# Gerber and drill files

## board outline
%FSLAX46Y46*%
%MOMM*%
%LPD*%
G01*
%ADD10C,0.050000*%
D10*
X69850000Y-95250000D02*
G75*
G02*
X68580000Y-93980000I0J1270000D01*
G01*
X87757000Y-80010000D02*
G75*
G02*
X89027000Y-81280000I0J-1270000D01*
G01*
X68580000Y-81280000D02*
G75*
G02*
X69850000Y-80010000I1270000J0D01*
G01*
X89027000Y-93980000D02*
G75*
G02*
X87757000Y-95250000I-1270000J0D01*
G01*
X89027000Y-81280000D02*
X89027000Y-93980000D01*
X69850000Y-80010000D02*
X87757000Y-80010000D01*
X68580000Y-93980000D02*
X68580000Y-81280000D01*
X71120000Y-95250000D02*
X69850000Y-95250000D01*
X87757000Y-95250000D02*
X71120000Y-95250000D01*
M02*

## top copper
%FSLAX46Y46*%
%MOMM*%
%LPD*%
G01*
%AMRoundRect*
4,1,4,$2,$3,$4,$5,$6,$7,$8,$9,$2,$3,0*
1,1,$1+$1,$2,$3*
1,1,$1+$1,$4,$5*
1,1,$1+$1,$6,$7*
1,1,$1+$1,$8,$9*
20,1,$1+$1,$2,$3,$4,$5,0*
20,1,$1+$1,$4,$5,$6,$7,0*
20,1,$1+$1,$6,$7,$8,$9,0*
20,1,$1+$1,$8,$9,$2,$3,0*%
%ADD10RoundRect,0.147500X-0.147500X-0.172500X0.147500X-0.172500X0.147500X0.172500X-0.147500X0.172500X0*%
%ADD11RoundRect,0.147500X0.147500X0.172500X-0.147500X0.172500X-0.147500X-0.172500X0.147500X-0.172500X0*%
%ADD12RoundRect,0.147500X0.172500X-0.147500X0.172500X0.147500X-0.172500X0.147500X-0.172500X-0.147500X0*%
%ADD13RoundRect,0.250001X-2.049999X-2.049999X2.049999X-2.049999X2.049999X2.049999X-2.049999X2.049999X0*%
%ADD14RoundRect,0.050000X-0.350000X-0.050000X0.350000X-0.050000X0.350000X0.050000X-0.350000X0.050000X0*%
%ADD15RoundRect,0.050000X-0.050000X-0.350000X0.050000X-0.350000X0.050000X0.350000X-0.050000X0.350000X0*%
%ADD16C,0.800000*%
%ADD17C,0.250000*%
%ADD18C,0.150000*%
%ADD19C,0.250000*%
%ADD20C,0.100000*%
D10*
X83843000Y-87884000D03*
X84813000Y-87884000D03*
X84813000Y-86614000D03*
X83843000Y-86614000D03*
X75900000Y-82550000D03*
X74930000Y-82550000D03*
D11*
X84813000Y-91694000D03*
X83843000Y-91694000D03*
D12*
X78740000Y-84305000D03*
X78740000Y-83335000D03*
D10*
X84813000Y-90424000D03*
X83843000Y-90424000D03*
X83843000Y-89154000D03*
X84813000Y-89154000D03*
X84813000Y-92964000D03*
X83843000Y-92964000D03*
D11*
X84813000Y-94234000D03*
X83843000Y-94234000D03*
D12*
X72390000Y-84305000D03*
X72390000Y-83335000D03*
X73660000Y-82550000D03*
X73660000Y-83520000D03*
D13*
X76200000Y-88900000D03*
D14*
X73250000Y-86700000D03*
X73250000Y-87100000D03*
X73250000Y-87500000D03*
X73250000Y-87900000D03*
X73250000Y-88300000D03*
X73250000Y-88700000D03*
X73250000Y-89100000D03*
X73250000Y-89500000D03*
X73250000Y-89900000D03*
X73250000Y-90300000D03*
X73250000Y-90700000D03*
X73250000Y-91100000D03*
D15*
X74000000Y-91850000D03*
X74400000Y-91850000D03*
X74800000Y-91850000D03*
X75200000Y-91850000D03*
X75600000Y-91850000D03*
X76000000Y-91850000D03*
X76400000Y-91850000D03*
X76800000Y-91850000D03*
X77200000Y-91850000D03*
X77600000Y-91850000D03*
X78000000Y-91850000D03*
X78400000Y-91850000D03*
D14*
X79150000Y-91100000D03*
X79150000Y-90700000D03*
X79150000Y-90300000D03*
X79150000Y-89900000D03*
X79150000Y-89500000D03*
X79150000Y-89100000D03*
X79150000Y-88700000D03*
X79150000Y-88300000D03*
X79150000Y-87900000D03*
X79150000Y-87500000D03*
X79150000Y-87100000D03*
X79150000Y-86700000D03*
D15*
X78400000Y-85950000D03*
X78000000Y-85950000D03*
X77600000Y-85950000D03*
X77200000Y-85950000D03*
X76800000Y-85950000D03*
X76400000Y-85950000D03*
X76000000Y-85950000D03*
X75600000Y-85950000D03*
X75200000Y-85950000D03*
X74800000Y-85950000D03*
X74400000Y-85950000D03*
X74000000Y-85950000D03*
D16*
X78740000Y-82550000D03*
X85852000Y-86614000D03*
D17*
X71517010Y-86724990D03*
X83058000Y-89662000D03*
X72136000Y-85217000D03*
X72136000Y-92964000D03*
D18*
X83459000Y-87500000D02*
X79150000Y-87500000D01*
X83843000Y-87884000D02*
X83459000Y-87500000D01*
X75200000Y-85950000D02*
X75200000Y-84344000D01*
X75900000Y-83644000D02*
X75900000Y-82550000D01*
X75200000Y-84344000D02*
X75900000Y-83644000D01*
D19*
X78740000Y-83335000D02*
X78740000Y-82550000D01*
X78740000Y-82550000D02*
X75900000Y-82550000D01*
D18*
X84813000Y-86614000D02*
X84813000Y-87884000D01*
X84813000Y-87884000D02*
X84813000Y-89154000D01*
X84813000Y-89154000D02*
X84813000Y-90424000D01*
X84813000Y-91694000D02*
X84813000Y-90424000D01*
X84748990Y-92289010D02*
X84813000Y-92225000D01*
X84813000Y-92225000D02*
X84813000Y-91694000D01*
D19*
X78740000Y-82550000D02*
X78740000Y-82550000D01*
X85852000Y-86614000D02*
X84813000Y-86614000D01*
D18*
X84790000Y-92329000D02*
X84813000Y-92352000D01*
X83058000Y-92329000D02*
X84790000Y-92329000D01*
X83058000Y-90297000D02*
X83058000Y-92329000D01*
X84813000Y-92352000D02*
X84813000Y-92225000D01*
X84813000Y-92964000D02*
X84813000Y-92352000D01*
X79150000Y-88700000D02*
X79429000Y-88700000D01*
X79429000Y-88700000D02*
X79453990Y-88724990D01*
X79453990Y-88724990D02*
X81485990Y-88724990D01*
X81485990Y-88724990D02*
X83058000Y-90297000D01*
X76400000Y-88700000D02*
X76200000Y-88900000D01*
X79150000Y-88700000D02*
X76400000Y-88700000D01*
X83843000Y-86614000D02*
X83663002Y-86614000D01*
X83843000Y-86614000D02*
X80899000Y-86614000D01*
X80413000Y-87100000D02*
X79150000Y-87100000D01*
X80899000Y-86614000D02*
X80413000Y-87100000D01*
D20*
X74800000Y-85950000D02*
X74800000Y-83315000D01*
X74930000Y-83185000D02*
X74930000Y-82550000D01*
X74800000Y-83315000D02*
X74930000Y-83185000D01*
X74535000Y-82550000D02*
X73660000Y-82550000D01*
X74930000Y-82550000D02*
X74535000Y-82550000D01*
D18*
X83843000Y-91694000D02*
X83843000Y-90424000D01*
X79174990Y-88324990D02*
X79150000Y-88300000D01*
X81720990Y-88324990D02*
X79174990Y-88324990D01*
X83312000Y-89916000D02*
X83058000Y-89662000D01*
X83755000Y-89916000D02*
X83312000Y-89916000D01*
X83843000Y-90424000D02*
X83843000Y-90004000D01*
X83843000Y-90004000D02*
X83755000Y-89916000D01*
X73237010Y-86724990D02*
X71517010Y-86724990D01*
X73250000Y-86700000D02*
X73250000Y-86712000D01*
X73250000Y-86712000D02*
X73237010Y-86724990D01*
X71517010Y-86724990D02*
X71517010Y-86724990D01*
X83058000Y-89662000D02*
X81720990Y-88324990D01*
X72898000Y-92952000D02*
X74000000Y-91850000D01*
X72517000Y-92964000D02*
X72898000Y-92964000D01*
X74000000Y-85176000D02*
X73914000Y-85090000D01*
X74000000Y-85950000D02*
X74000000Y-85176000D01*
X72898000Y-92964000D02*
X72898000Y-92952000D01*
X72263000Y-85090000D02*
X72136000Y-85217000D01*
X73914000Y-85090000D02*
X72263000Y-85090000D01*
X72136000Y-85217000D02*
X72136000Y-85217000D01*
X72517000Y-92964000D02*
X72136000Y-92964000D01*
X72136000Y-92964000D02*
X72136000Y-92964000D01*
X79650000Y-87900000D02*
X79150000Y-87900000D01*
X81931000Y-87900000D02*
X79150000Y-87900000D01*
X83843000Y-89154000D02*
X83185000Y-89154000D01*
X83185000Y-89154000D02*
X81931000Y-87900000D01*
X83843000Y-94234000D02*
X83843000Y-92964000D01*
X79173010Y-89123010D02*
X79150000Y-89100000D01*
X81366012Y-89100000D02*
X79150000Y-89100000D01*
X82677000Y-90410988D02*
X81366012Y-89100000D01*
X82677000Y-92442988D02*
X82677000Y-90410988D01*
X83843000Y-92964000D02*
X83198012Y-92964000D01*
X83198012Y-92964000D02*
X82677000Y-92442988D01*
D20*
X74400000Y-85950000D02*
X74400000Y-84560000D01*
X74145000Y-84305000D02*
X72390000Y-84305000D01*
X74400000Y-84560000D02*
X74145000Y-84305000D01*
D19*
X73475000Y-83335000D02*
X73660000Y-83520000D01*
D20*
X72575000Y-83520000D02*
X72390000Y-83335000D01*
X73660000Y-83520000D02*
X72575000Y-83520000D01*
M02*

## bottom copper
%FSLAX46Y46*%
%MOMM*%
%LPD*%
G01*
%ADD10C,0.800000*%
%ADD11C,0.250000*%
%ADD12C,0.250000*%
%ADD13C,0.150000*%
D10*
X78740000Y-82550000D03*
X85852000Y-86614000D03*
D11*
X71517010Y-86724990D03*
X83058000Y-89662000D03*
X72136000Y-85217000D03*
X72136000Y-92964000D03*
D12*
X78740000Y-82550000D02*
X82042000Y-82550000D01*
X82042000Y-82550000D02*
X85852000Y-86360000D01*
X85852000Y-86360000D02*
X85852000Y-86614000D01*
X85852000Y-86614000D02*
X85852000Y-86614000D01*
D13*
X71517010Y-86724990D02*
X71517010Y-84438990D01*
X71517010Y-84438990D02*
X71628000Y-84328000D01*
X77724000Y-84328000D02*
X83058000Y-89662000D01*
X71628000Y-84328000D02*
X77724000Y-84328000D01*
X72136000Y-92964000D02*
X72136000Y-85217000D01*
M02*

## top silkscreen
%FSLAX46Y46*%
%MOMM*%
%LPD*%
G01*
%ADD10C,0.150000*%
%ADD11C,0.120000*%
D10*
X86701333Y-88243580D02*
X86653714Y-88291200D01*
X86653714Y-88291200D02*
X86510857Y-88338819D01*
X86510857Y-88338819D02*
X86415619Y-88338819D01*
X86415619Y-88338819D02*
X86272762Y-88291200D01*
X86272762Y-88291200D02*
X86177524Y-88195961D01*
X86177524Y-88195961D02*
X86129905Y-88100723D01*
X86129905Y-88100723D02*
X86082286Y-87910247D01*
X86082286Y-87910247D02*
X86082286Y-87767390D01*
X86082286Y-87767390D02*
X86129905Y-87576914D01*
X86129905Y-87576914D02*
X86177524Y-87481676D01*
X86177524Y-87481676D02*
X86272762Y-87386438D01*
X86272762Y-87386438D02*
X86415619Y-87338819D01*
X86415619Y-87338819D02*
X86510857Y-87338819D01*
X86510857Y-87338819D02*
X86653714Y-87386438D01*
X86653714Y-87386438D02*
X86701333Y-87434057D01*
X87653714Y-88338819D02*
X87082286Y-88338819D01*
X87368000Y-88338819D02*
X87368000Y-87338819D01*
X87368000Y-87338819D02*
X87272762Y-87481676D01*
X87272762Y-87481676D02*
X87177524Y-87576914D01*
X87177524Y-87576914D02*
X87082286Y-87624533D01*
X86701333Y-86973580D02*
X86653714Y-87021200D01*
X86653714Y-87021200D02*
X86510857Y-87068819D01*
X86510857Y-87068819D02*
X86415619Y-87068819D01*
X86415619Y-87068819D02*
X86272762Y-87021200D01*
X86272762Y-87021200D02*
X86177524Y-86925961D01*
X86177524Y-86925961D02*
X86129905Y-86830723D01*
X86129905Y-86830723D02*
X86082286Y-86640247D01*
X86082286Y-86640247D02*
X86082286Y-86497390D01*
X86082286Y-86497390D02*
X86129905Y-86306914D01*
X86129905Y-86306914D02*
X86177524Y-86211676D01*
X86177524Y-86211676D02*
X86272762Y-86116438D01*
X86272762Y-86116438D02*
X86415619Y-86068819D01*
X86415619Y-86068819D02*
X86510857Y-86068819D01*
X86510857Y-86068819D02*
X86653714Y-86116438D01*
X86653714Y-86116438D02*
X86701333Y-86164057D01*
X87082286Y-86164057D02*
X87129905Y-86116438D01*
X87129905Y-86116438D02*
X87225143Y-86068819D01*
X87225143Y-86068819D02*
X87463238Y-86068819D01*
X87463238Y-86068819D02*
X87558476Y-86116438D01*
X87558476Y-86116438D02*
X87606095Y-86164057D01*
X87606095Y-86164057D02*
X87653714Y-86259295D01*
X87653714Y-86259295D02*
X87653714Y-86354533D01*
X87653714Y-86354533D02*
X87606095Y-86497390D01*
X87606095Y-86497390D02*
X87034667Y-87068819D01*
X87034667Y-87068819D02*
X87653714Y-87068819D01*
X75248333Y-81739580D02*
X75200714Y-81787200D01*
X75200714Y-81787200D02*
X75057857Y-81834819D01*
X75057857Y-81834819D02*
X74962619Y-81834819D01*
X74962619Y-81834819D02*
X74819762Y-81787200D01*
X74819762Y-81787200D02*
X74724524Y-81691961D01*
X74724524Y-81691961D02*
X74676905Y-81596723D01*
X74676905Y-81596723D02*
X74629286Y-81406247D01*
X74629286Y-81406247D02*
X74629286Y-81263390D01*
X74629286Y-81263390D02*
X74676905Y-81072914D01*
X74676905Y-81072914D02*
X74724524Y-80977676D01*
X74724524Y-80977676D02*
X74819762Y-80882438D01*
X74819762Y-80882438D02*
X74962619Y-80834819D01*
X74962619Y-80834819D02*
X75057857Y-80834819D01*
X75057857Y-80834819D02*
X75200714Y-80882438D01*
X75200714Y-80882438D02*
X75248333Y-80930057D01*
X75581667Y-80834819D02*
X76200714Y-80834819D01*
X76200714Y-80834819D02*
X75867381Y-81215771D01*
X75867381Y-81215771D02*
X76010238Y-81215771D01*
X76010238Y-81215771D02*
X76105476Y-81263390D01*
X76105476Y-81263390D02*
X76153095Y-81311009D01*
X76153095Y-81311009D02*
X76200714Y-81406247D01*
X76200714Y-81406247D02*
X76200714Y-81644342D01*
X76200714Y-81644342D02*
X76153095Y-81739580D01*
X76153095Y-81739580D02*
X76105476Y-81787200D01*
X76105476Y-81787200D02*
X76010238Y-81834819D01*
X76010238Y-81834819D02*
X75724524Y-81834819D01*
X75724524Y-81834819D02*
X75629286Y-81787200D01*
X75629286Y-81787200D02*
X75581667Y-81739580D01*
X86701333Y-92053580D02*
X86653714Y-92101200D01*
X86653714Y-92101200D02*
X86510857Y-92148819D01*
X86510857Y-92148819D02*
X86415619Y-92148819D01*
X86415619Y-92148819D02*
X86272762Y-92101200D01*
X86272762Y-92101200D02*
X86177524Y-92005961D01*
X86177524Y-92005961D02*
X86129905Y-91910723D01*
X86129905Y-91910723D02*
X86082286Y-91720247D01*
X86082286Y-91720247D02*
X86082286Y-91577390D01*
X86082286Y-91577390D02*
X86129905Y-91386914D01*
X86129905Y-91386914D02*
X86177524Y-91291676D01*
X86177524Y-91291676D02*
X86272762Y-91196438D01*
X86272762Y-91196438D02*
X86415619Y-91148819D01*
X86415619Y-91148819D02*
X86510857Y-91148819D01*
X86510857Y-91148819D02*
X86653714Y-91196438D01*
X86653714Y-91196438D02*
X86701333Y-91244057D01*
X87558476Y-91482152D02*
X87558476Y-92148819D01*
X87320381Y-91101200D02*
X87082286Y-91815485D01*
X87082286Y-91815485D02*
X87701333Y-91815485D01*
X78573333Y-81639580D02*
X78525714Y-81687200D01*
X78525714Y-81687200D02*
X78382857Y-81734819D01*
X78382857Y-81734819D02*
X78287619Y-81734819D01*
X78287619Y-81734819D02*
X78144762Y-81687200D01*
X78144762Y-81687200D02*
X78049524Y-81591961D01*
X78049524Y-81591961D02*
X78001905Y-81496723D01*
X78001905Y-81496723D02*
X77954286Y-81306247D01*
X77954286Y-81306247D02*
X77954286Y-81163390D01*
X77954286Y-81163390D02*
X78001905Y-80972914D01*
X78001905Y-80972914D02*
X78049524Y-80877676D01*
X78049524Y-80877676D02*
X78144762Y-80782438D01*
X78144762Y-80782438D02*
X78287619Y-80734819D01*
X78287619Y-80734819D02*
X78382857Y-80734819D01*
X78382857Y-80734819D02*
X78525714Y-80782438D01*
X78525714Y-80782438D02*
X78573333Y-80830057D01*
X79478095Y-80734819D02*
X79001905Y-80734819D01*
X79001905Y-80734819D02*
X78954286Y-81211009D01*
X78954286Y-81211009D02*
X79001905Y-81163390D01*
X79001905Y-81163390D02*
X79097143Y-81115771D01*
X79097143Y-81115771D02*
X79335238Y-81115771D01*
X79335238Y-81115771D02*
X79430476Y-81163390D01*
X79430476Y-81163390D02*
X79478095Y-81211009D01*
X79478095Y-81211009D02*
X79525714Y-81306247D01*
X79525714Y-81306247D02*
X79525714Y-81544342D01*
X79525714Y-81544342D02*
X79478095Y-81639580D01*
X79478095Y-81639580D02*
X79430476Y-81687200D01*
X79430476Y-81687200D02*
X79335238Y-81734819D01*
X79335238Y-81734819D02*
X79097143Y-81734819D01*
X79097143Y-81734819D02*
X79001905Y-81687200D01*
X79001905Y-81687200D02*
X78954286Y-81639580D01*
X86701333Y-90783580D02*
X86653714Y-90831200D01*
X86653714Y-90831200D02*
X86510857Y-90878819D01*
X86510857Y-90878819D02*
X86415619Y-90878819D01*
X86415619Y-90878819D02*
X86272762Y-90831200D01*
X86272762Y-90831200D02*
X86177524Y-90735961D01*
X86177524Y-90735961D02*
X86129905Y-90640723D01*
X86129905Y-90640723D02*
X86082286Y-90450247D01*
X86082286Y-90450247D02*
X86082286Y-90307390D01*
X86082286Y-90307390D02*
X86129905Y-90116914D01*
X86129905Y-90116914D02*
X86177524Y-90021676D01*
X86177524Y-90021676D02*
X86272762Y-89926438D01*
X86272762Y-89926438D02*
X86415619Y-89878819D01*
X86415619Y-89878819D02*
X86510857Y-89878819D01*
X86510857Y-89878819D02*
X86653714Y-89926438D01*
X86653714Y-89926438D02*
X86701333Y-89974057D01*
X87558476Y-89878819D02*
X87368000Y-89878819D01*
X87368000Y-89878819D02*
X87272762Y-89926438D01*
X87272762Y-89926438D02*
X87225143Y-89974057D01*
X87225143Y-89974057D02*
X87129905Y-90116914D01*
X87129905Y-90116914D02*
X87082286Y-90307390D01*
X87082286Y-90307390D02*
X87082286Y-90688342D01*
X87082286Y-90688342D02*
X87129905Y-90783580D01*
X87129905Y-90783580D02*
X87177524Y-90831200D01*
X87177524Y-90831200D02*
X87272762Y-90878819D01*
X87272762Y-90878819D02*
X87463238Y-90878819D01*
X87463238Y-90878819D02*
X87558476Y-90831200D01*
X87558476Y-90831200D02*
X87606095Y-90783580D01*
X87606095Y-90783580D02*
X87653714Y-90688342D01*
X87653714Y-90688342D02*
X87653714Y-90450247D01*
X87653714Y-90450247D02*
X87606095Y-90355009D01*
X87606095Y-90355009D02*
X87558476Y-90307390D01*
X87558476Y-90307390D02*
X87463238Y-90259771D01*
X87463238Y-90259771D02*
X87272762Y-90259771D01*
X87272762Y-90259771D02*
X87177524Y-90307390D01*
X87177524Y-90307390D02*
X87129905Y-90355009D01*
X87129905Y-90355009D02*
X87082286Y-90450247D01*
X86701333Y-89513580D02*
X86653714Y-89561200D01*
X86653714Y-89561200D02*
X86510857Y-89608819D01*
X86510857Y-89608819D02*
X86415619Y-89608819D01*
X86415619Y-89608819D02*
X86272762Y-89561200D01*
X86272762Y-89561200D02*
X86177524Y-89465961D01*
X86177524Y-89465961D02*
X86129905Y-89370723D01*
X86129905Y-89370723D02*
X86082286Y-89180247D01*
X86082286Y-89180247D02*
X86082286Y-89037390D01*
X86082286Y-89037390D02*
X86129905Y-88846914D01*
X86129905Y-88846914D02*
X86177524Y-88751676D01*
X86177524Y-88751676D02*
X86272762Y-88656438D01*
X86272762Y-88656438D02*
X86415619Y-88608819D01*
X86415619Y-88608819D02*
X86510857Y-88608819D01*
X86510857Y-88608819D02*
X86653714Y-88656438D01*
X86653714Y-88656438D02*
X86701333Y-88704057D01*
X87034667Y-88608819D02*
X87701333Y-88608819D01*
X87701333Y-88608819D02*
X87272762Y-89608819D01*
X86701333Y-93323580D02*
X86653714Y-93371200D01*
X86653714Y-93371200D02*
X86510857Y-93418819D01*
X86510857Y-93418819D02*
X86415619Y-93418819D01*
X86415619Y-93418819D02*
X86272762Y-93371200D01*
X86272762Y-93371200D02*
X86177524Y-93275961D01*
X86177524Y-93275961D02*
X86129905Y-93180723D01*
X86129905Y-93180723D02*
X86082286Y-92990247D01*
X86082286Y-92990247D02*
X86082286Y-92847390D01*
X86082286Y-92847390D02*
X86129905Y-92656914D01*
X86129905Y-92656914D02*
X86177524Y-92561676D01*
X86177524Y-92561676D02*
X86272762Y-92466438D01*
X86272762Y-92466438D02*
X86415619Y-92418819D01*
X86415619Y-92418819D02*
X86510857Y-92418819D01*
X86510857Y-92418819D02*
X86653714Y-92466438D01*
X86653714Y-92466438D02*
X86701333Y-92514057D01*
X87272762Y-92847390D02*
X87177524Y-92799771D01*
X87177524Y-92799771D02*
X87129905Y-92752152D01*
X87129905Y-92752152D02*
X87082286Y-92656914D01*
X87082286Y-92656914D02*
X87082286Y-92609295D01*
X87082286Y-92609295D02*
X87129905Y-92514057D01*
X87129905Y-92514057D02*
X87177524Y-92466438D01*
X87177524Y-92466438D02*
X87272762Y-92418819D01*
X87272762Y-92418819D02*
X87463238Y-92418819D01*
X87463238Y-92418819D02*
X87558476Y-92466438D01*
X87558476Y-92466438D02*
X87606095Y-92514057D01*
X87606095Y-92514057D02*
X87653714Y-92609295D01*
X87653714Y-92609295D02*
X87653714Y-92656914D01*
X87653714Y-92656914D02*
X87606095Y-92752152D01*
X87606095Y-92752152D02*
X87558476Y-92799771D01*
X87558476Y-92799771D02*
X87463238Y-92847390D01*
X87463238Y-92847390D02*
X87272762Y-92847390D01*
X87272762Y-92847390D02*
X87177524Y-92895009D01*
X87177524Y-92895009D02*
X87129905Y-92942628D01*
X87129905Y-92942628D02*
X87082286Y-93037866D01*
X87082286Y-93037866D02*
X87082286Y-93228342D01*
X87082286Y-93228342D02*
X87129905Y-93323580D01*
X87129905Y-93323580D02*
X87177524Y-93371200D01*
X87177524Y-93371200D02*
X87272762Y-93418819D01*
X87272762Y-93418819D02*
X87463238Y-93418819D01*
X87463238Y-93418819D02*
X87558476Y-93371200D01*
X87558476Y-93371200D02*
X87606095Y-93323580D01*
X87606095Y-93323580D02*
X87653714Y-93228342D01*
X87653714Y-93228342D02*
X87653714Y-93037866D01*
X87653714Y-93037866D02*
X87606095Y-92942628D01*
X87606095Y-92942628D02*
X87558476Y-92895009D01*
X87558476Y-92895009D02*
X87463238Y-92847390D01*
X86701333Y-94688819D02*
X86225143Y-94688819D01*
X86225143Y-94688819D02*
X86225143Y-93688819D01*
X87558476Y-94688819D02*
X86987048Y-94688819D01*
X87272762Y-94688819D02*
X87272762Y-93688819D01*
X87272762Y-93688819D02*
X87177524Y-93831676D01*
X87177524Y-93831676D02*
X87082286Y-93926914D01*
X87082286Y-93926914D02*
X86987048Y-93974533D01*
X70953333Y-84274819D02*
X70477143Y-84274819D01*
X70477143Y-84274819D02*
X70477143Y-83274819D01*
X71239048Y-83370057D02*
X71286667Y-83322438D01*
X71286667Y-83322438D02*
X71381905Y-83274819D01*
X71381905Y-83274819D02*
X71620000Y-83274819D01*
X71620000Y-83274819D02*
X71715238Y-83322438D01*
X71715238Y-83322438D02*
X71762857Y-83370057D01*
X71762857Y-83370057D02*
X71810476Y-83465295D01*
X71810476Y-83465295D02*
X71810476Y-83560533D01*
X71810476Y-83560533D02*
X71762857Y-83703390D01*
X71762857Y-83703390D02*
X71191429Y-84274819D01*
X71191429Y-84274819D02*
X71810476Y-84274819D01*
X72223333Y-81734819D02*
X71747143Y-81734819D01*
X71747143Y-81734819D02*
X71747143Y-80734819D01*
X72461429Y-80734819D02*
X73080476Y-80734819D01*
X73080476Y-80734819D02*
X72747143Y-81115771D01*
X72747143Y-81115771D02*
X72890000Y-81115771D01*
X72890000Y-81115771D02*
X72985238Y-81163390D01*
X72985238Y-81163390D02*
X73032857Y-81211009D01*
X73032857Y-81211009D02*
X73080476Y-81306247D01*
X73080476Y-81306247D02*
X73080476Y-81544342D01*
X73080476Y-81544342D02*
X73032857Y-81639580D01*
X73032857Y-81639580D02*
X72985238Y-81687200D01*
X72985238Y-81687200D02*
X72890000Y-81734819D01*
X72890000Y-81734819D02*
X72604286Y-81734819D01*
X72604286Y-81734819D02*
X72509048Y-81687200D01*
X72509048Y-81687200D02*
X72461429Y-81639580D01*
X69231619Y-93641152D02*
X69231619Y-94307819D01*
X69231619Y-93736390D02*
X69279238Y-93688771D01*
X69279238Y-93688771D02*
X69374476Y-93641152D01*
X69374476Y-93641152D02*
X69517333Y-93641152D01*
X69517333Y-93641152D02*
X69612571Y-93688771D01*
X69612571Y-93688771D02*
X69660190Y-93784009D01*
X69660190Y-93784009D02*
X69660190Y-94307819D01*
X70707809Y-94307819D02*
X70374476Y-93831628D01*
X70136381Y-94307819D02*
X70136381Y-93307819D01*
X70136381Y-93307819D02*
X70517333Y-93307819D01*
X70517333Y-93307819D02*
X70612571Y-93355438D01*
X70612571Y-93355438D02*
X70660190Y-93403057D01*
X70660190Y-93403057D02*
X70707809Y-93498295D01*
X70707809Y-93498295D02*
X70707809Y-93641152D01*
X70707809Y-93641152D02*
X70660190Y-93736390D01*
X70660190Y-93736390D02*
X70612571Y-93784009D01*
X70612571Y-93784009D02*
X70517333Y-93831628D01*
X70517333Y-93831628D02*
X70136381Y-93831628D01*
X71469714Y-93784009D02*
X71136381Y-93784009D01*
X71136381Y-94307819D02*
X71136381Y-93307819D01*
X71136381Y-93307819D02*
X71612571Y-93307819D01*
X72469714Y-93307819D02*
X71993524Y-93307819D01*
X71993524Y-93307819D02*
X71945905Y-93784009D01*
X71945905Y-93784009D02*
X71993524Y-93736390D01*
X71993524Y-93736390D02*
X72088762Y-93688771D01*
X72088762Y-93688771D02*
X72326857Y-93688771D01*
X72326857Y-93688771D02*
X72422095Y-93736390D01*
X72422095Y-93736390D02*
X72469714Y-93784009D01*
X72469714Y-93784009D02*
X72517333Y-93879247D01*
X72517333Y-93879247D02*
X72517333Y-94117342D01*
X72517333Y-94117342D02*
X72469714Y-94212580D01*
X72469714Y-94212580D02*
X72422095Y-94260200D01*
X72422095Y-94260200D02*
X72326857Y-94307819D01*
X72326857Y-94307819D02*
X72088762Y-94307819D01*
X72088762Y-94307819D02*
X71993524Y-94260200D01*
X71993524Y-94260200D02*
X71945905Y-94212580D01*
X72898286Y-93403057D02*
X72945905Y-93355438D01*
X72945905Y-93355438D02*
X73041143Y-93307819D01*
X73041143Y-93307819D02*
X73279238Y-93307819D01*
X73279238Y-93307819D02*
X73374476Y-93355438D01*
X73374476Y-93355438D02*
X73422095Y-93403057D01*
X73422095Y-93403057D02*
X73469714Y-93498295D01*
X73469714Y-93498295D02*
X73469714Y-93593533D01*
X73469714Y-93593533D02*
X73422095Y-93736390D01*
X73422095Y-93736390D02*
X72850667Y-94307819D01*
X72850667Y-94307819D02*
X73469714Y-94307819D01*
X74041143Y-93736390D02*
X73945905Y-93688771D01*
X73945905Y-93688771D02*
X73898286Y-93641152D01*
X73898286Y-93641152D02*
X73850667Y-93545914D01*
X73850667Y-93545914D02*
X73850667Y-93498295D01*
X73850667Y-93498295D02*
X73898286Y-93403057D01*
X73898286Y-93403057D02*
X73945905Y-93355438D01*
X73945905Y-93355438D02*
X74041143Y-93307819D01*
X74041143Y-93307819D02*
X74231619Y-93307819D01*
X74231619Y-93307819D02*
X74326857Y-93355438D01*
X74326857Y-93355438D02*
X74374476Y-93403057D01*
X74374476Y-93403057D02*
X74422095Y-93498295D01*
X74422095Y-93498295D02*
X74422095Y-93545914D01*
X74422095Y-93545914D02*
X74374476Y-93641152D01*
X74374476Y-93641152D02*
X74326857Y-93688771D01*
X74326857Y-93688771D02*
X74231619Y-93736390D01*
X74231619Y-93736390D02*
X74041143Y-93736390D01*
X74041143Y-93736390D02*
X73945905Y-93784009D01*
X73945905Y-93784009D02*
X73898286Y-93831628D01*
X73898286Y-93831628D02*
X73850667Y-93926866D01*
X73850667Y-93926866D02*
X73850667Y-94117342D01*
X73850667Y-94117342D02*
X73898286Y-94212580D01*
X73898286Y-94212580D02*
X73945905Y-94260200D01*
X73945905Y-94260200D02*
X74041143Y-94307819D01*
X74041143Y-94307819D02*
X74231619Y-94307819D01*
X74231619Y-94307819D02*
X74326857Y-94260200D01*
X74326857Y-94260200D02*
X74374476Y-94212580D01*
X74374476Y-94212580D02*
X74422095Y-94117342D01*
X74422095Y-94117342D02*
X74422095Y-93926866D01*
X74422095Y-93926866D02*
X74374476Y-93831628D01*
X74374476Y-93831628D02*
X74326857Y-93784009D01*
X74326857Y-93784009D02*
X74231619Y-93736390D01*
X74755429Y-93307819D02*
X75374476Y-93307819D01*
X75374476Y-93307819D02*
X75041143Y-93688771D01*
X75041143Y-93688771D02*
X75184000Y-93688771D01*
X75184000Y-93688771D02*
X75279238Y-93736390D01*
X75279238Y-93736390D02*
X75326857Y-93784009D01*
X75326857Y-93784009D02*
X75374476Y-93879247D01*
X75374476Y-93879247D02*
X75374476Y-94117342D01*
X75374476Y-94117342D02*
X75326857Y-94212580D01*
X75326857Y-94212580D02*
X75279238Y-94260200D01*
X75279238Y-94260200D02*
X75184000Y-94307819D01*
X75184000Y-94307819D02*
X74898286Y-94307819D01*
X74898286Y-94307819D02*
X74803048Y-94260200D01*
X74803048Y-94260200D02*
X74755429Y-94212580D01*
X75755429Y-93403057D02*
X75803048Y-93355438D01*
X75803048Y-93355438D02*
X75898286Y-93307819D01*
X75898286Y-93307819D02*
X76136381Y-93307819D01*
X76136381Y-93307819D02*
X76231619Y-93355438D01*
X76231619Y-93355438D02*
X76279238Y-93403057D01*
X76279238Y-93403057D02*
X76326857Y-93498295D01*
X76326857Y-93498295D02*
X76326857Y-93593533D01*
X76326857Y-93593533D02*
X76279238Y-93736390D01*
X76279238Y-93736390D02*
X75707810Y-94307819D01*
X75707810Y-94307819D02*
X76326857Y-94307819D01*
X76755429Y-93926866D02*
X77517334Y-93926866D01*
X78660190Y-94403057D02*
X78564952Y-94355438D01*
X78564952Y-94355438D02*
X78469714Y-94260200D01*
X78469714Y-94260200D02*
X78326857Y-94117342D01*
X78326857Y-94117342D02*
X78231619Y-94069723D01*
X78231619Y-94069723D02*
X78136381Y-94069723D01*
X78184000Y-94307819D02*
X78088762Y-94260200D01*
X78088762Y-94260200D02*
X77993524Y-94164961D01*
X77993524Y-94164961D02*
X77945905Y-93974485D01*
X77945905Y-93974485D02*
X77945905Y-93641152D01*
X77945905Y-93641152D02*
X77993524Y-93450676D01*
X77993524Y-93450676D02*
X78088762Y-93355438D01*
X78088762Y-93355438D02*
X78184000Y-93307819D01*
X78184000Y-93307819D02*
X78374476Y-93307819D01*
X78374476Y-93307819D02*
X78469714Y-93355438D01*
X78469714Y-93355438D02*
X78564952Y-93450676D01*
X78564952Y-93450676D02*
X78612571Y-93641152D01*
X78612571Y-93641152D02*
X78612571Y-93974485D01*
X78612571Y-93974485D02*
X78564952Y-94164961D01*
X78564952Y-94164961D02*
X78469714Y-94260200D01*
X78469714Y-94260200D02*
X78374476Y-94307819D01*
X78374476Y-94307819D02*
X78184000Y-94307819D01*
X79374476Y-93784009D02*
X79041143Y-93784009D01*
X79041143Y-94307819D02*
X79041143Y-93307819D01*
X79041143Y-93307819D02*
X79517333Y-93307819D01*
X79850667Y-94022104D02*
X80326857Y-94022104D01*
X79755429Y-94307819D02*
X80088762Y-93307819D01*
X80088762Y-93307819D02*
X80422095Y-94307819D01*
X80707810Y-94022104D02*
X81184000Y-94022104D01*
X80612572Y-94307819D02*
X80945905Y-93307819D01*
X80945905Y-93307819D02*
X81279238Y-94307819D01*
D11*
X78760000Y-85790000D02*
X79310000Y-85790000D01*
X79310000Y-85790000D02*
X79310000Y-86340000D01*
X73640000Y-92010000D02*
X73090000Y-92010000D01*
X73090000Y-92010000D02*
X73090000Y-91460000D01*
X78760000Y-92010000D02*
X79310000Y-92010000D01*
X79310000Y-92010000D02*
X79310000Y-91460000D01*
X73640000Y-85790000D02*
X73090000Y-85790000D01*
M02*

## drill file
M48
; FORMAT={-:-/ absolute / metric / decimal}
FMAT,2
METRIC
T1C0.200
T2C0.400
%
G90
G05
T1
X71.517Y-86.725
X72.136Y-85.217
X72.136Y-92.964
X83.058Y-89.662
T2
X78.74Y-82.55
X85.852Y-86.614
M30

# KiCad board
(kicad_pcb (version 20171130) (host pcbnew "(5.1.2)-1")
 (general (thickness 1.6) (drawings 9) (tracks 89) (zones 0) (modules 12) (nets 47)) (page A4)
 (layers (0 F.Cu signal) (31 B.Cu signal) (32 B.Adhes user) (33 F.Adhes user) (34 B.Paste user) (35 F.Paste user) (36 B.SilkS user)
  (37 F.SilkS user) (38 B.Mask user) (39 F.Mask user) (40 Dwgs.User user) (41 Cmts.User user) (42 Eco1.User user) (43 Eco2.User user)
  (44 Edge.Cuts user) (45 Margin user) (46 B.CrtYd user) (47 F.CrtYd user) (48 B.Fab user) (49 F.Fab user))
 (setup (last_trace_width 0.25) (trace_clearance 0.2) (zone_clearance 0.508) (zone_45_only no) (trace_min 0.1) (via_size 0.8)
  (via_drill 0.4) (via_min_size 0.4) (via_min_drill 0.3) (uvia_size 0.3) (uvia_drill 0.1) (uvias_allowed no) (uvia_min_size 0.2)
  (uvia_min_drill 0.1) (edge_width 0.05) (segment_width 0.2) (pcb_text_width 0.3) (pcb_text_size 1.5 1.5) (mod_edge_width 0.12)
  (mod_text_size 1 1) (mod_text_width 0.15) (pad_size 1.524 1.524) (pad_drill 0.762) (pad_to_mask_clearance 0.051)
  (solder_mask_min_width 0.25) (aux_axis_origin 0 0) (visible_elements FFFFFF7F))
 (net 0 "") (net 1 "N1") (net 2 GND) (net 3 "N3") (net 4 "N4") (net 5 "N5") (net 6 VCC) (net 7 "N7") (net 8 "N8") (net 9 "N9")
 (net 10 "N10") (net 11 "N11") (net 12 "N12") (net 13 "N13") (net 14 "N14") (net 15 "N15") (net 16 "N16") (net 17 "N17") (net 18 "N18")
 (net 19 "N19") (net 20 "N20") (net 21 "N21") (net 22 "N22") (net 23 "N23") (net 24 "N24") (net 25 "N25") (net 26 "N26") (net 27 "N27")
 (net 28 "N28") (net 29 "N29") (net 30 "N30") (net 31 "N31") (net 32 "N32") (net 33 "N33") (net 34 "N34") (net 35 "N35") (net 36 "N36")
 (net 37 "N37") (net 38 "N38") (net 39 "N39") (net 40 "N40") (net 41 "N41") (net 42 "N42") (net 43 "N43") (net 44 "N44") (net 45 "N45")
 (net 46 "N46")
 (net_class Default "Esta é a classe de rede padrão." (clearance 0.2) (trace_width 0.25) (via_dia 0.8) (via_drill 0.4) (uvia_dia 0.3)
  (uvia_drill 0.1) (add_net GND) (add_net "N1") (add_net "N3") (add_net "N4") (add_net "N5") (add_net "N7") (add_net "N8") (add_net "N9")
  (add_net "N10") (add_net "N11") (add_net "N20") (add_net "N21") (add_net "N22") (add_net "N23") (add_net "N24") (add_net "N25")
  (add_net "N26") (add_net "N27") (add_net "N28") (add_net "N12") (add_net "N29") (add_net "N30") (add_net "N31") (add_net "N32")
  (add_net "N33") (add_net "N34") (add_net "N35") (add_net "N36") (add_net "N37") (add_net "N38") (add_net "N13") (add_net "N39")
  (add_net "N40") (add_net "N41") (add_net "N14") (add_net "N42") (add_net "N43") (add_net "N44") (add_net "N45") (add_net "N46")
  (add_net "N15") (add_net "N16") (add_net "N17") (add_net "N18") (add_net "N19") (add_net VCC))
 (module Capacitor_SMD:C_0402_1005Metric (layer F.Cu) (at 84.328 87.884)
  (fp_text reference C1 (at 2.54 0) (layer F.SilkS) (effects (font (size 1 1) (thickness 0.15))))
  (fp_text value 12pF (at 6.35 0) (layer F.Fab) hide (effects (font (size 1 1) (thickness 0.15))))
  (pad 1 smd roundrect (at -0.485 0) (size 0.59 0.64) (layers F.Cu F.Paste F.Mask) (roundrect_rratio 0.25) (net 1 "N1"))
  (pad 2 smd roundrect (at 0.485 0) (size 0.59 0.64) (layers F.Cu F.Paste F.Mask) (roundrect_rratio 0.25) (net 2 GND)))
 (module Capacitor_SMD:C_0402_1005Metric (layer F.Cu) (at 84.328 86.614)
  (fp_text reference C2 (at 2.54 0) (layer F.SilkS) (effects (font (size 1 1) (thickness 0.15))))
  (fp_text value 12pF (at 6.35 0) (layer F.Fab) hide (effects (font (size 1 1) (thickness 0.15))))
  (pad 2 smd roundrect (at 0.485 0) (size 0.59 0.64) (layers F.Cu F.Paste F.Mask) (roundrect_rratio 0.25) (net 2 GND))
  (pad 1 smd roundrect (at -0.485 0) (size 0.59 0.64) (layers F.Cu F.Paste F.Mask) (roundrect_rratio 0.25) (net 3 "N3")))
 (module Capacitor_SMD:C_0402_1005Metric (layer F.Cu) (at 75.415 82.55)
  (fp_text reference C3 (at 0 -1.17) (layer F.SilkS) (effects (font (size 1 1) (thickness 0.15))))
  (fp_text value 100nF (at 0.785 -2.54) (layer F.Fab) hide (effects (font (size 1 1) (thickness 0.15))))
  (pad 2 smd roundrect (at 0.485 0) (size 0.59 0.64) (layers F.Cu F.Paste F.Mask) (roundrect_rratio 0.25) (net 2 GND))
  (pad 1 smd roundrect (at -0.485 0) (size 0.59 0.64) (layers F.Cu F.Paste F.Mask) (roundrect_rratio 0.25) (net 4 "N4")))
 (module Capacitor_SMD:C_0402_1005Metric (layer F.Cu) (at 84.328 91.694 180)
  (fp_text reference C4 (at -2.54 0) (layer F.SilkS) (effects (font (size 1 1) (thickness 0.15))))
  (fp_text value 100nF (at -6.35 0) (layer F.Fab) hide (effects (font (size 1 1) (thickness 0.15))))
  (pad 1 smd roundrect (at -0.485 0 180) (size 0.59 0.64) (layers F.Cu F.Paste F.Mask) (roundrect_rratio 0.25) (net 2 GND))
  (pad 2 smd roundrect (at 0.485 0 180) (size 0.59 0.64) (layers F.Cu F.Paste F.Mask) (roundrect_rratio 0.25) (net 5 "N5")))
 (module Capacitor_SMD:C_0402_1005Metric (layer F.Cu) (at 78.74 83.82 90)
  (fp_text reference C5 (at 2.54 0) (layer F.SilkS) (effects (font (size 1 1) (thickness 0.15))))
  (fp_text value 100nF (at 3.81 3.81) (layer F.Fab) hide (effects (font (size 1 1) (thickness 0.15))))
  (pad 1 smd roundrect (at -0.485 0 90) (size 0.59 0.64) (layers F.Cu F.Paste F.Mask) (roundrect_rratio 0.25) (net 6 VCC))
  (pad 2 smd roundrect (at 0.485 0 90) (size 0.59 0.64) (layers F.Cu F.Paste F.Mask) (roundrect_rratio 0.25) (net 2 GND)))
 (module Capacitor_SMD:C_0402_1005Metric (layer F.Cu) (at 84.328 90.424)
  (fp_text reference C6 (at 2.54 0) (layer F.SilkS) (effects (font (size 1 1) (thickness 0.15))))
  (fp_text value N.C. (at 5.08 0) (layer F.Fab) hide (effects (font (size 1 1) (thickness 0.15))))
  (pad 2 smd roundrect (at 0.485 0) (size 0.59 0.64) (layers F.Cu F.Paste F.Mask) (roundrect_rratio 0.25) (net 2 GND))
  (pad 1 smd roundrect (at -0.485 0) (size 0.59 0.64) (layers F.Cu F.Paste F.Mask) (roundrect_rratio 0.25) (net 5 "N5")))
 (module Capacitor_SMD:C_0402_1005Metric (layer F.Cu) (at 84.328 89.154)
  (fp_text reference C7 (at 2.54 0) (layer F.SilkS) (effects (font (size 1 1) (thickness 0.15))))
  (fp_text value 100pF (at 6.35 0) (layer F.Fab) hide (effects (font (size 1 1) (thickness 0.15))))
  (pad 1 smd roundrect (at -0.485 0) (size 0.59 0.64) (layers F.Cu F.Paste F.Mask) (roundrect_rratio 0.25) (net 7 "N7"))
  (pad 2 smd roundrect (at 0.485 0) (size 0.59 0.64) (layers F.Cu F.Paste F.Mask) (roundrect_rratio 0.25) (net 2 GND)))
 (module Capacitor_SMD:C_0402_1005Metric (layer F.Cu) (at 84.328 92.964)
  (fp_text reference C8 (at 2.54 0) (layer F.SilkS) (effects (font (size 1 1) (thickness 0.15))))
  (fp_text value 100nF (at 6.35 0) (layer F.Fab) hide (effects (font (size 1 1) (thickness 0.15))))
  (pad 2 smd roundrect (at 0.485 0) (size 0.59 0.64) (layers F.Cu F.Paste F.Mask) (roundrect_rratio 0.25) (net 2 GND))
  (pad 1 smd roundrect (at -0.485 0) (size 0.59 0.64) (layers F.Cu F.Paste F.Mask) (roundrect_rratio 0.25) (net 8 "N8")))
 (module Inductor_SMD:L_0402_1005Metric (layer F.Cu) (at 84.328 94.234 180)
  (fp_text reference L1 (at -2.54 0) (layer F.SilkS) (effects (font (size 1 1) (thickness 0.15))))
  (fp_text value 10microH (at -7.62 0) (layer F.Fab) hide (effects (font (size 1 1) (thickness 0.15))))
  (pad 1 smd roundrect (at -0.485 0 180) (size 0.59 0.64) (layers F.Cu F.Paste F.Mask) (roundrect_rratio 0.25) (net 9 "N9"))
  (pad 2 smd roundrect (at 0.485 0 180) (size 0.59 0.64) (layers F.Cu F.Paste F.Mask) (roundrect_rratio 0.25) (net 8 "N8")))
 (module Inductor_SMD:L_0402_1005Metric (layer F.Cu) (at 72.39 83.82 90)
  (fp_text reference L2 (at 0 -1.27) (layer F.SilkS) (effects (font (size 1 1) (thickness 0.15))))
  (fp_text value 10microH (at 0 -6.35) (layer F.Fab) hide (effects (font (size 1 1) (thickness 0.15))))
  (pad 1 smd roundrect (at -0.485 0 90) (size 0.59 0.64) (layers F.Cu F.Paste F.Mask) (roundrect_rratio 0.25) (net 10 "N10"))
  (pad 2 smd roundrect (at 0.485 0 90) (size 0.59 0.64) (layers F.Cu F.Paste F.Mask) (roundrect_rratio 0.25) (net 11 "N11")))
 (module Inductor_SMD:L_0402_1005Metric (layer F.Cu) (at 73.66 83.035 90)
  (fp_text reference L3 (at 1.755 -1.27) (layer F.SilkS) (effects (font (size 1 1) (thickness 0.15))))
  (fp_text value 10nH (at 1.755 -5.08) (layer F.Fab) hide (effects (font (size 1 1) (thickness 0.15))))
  (pad 2 smd roundrect (at 0.485 0 90) (size 0.59 0.64) (layers F.Cu F.Paste F.Mask) (roundrect_rratio 0.25) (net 4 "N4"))
  (pad 1 smd roundrect (at -0.485 0 90) (size 0.59 0.64) (layers F.Cu F.Paste F.Mask) (roundrect_rratio 0.25) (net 11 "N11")))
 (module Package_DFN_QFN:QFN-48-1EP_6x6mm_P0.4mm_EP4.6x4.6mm (layer F.Cu) (at 76.2 88.9)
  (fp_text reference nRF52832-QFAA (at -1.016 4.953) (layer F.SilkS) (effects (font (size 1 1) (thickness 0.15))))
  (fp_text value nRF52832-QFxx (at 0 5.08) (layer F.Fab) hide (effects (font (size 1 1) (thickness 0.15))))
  (fp_line (start 2.56 -3.11) (end 3.11 -3.11) (layer F.SilkS) (width 0.12))
  (fp_line (start 3.11 -3.11) (end 3.11 -2.56) (layer F.SilkS) (width 0.12))
  (fp_line (start -2.56 3.11) (end -3.11 3.11) (layer F.SilkS) (width 0.12))
  (fp_line (start -3.11 3.11) (end -3.11 2.56) (layer F.SilkS) (width 0.12))
  (fp_line (start 2.56 3.11) (end 3.11 3.11) (layer F.SilkS) (width 0.12))
  (fp_line (start 3.11 3.11) (end 3.11 2.56) (layer F.SilkS) (width 0.12))
  (fp_line (start -2.56 -3.11) (end -3.11 -3.11) (layer F.SilkS) (width 0.12))
  (pad 49 smd roundrect (at 0 0) (size 4.6 4.6) (layers F.Cu F.Mask) (roundrect_rratio 0.054348) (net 2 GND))
  (pad "" smd roundrect (at -1.53 -1.53) (size 1.24 1.24) (layers F.Paste) (roundrect_rratio 0.201613))
  (pad "" smd roundrect (at -1.53 0) (size 1.24 1.24) (layers F.Paste) (roundrect_rratio 0.201613))
  (pad "" smd roundrect (at -1.53 1.53) (size 1.24 1.24) (layers F.Paste) (roundrect_rratio 0.201613))
  (pad "" smd roundrect (at 0 -1.53) (size 1.24 1.24) (layers F.Paste) (roundrect_rratio 0.201613))
  (pad "" smd roundrect (at 0 0) (size 1.24 1.24) (layers F.Paste) (roundrect_rratio 0.201613))
  (pad "" smd roundrect (at 0 1.53) (size 1.24 1.24) (layers F.Paste) (roundrect_rratio 0.201613))
  (pad "" smd roundrect (at 1.53 -1.53) (size 1.24 1.24) (layers F.Paste) (roundrect_rratio 0.201613))
  (pad "" smd roundrect (at 1.53 0) (size 1.24 1.24) (layers F.Paste) (roundrect_rratio 0.201613))
  (pad "" smd roundrect (at 1.53 1.53) (size 1.24 1.24) (layers F.Paste) (roundrect_rratio 0.201613))
  (pad 1 smd roundrect (at -2.95 -2.2) (size 0.8 0.2) (layers F.Cu F.Paste F.Mask) (roundrect_rratio 0.25) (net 5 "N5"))
  (pad 2 smd roundrect (at -2.95 -1.8) (size 0.8 0.2) (layers F.Cu F.Paste F.Mask) (roundrect_rratio 0.25) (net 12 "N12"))
  (pad 3 smd roundrect (at -2.95 -1.4) (size 0.8 0.2) (layers F.Cu F.Paste F.Mask) (roundrect_rratio 0.25) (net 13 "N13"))
  (pad 4 smd roundrect (at -2.95 -1) (size 0.8 0.2) (layers F.Cu F.Paste F.Mask) (roundrect_rratio 0.25) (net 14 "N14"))
  (pad 5 smd roundrect (at -2.95 -0.6) (size 0.8 0.2) (layers F.Cu F.Paste F.Mask) (roundrect_rratio 0.25) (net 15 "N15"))
  (pad 6 smd roundrect (at -2.95 -0.2) (size 0.8 0.2) (layers F.Cu F.Paste F.Mask) (roundrect_rratio 0.25) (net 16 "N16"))
  (pad 7 smd roundrect (at -2.95 0.2) (size 0.8 0.2) (layers F.Cu F.Paste F.Mask) (roundrect_rratio 0.25) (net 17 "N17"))
  (pad 8 smd roundrect (at -2.95 0.6) (size 0.8 0.2) (layers F.Cu F.Paste F.Mask) (roundrect_rratio 0.25) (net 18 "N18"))
  (pad 9 smd roundrect (at -2.95 1) (size 0.8 0.2) (layers F.Cu F.Paste F.Mask) (roundrect_rratio 0.25) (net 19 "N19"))
  (pad 10 smd roundrect (at -2.95 1.4) (size 0.8 0.2) (layers F.Cu F.Paste F.Mask) (roundrect_rratio 0.25) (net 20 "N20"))
  (pad 11 smd roundrect (at -2.95 1.8) (size 0.8 0.2) (layers F.Cu F.Paste F.Mask) (roundrect_rratio 0.25) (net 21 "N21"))
  (pad 12 smd roundrect (at -2.95 2.2) (size 0.8 0.2) (layers F.Cu F.Paste F.Mask) (roundrect_rratio 0.25) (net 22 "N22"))
  (pad 13 smd roundrect (at -2.2 2.95) (size 0.2 0.8) (layers F.Cu F.Paste F.Mask) (roundrect_rratio 0.25) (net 6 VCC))
  (pad 14 smd roundrect (at -1.8 2.95) (size 0.2 0.8) (layers F.Cu F.Paste F.Mask) (roundrect_rratio 0.25) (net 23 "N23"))
  (pad 15 smd roundrect (at -1.4 2.95) (size 0.2 0.8) (layers F.Cu F.Paste F.Mask) (roundrect_rratio 0.25) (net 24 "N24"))
  (pad 16 smd roundrect (at -1 2.95) (size 0.2 0.8) (layers F.Cu F.Paste F.Mask) (roundrect_rratio 0.25) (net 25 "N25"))
  (pad 17 smd roundrect (at -0.6 2.95) (size 0.2 0.8) (layers F.Cu F.Paste F.Mask) (roundrect_rratio 0.25) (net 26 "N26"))
  (pad 18 smd roundrect (at -0.2 2.95) (size 0.2 0.8) (layers F.Cu F.Paste F.Mask) (roundrect_rratio 0.25) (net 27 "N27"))
  (pad 19 smd roundrect (at 0.2 2.95) (size 0.2 0.8) (layers F.Cu F.Paste F.Mask) (roundrect_rratio 0.25) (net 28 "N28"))
  (pad 20 smd roundrect (at 0.6 2.95) (size 0.2 0.8) (layers F.Cu F.Paste F.Mask) (roundrect_rratio 0.25) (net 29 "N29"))
  (pad 21 smd roundrect (at 1 2.95) (size 0.2 0.8) (layers F.Cu F.Paste F.Mask) (roundrect_rratio 0.25) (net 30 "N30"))
  (pad 22 smd roundrect (at 1.4 2.95) (size 0.2 0.8) (layers F.Cu F.Paste F.Mask) (roundrect_rratio 0.25) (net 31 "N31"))
  (pad 23 smd roundrect (at 1.8 2.95) (size 0.2 0.8) (layers F.Cu F.Paste F.Mask) (roundrect_rratio 0.25) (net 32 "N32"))
  (pad 24 smd roundrect (at 2.2 2.95) (size 0.2 0.8) (layers F.Cu F.Paste F.Mask) (roundrect_rratio 0.25) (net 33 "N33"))
  (pad 25 smd roundrect (at 2.95 2.2) (size 0.8 0.2) (layers F.Cu F.Paste F.Mask) (roundrect_rratio 0.25) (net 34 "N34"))
  (pad 26 smd roundrect (at 2.95 1.8) (size 0.8 0.2) (layers F.Cu F.Paste F.Mask) (roundrect_rratio 0.25) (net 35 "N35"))
  (pad 27 smd roundrect (at 2.95 1.4) (size 0.8 0.2) (layers F.Cu F.Paste F.Mask) (roundrect_rratio 0.25) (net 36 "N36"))
  (pad 28 smd roundrect (at 2.95 1) (size 0.8 0.2) (layers F.Cu F.Paste F.Mask) (roundrect_rratio 0.25) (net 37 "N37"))
  (pad 29 smd roundrect (at 2.95 0.6) (size 0.8 0.2) (layers F.Cu F.Paste F.Mask) (roundrect_rratio 0.25) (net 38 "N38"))
  (pad 30 smd roundrect (at 2.95 0.2) (size 0.8 0.2) (layers F.Cu F.Paste F.Mask) (roundrect_rratio 0.25) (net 8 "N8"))
  (pad 31 smd roundrect (at 2.95 -0.2) (size 0.8 0.2) (layers F.Cu F.Paste F.Mask) (roundrect_rratio 0.25) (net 2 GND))
  (pad 32 smd roundrect (at 2.95 -0.6) (size 0.8 0.2) (layers F.Cu F.Paste F.Mask) (roundrect_rratio 0.25) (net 5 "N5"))
  (pad 33 smd roundrect (at 2.95 -1) (size 0.8 0.2) (layers F.Cu F.Paste F.Mask) (roundrect_rratio 0.25) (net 7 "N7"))
  (pad 34 smd roundrect (at 2.95 -1.4) (size 0.8 0.2) (layers F.Cu F.Paste F.Mask) (roundrect_rratio 0.25) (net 1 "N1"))
  (pad 35 smd roundrect (at 2.95 -1.8) (size 0.8 0.2) (layers F.Cu F.Paste F.Mask) (roundrect_rratio 0.25) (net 3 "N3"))
  (pad 36 smd roundrect (at 2.95 -2.2) (size 0.8 0.2) (layers F.Cu F.Paste F.Mask) (roundrect_rratio 0.25) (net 6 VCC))
  (pad 37 smd roundrect (at 2.2 -2.95) (size 0.2 0.8) (layers F.Cu F.Paste F.Mask) (roundrect_rratio 0.25) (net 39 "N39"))
  (pad 38 smd roundrect (at 1.8 -2.95) (size 0.2 0.8) (layers F.Cu F.Paste F.Mask) (roundrect_rratio 0.25) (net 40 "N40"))
  (pad 39 smd roundrect (at 1.4 -2.95) (size 0.2 0.8) (layers F.Cu F.Paste F.Mask) (roundrect_rratio 0.25) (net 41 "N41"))
  (pad 40 smd roundrect (at 1 -2.95) (size 0.2 0.8) (layers F.Cu F.Paste F.Mask) (roundrect_rratio 0.25) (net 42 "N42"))
  (pad 41 smd roundrect (at 0.6 -2.95) (size 0.2 0.8) (layers F.Cu F.Paste F.Mask) (roundrect_rratio 0.25) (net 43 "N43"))
  (pad 42 smd roundrect (at 0.2 -2.95) (size 0.2 0.8) (layers F.Cu F.Paste F.Mask) (roundrect_rratio 0.25) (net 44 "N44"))
  (pad 43 smd roundrect (at -0.2 -2.95) (size 0.2 0.8) (layers F.Cu F.Paste F.Mask) (roundrect_rratio 0.25) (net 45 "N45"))
  (pad 44 smd roundrect (at -0.6 -2.95) (size 0.2 0.8) (layers F.Cu F.Paste F.Mask) (roundrect_rratio 0.25) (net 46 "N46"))
  (pad 45 smd roundrect (at -1 -2.95) (size 0.2 0.8) (layers F.Cu F.Paste F.Mask) (roundrect_rratio 0.25) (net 2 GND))
  (pad 46 smd roundrect (at -1.4 -2.95) (size 0.2 0.8) (layers F.Cu F.Paste F.Mask) (roundrect_rratio 0.25) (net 4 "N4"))
  (pad 47 smd roundrect (at -1.8 -2.95) (size 0.2 0.8) (layers F.Cu F.Paste F.Mask) (roundrect_rratio 0.25) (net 10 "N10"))
  (pad 48 smd roundrect (at -2.2 -2.95) (size 0.2 0.8) (layers F.Cu F.Paste F.Mask) (roundrect_rratio 0.25) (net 6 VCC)))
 (gr_arc (start 69.85 93.98) (end 68.58 93.98) (angle -90) (layer Edge.Cuts) (width 0.05))
 (gr_arc (start 87.757 81.28) (end 89.027 81.28) (angle -90) (layer Edge.Cuts) (width 0.05))
 (gr_arc (start 69.85 81.28) (end 69.85 80.01) (angle -90) (layer Edge.Cuts) (width 0.05))
 (gr_arc (start 87.757 93.98) (end 87.757 95.25) (angle -90) (layer Edge.Cuts) (width 0.05))
 (gr_line (start 89.027 81.28) (end 89.027 93.98) (layer Edge.Cuts) (width 0.05))
 (gr_line (start 69.85 80.01) (end 87.757 80.01) (layer Edge.Cuts) (width 0.05))
 (gr_line (start 68.58 93.98) (end 68.58 81.28) (layer Edge.Cuts) (width 0.05))
 (gr_line (start 71.12 95.25) (end 69.85 95.25) (layer Edge.Cuts) (width 0.05))
 (gr_line (start 87.757 95.25) (end 71.12 95.25) (layer Edge.Cuts) (width 0.05))
 (segment (start 83.459 87.5) (end 79.15 87.5) (width 0.15) (layer F.Cu) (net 1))
 (segment (start 83.843 87.884) (end 83.459 87.5) (width 0.15) (layer F.Cu) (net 1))
 (segment (start 75.2 85.95) (end 75.2 84.344) (width 0.15) (layer F.Cu) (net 2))
 (segment (start 75.9 83.644) (end 75.9 82.55) (width 0.15) (layer F.Cu) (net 2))
 (segment (start 75.2 84.344) (end 75.9 83.644) (width 0.15) (layer F.Cu) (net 2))
 (segment (start 78.74 83.335) (end 78.74 82.55) (width 0.25) (layer F.Cu) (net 2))
 (segment (start 78.74 82.55) (end 75.9 82.55) (width 0.25) (layer F.Cu) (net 2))
 (segment (start 84.813 86.614) (end 84.813 87.884) (width 0.15) (layer F.Cu) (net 2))
 (segment (start 84.813 87.884) (end 84.813 89.154) (width 0.15) (layer F.Cu) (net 2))
 (segment (start 84.813 89.154) (end 84.813 90.424) (width 0.15) (layer F.Cu) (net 2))
 (segment (start 84.813 91.694) (end 84.813 90.424) (width 0.15) (layer F.Cu) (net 2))
 (segment (start 84.74899 92.28901) (end 84.813 92.225) (width 0.15) (layer F.Cu) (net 2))
 (segment (start 84.813 92.225) (end 84.813 91.694) (width 0.15) (layer F.Cu) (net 2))
 (segment (start 78.74 82.55) (end 78.74 82.55) (width 0.25) (layer F.Cu) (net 2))
 (via (at 78.74 82.55) (size 0.8) (drill 0.4) (layers F.Cu B.Cu) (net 2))
 (segment (start 78.74 82.55) (end 82.042 82.55) (width 0.25) (layer B.Cu) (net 2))
 (segment (start 82.042 82.55) (end 85.852 86.36) (width 0.25) (layer B.Cu) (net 2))
 (segment (start 85.852 86.36) (end 85.852 86.614) (width 0.25) (layer B.Cu) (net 2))
 (segment (start 85.852 86.614) (end 85.852 86.614) (width 0.25) (layer B.Cu) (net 2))
 (via (at 85.852 86.614) (size 0.8) (drill 0.4) (layers F.Cu B.Cu) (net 2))
 (segment (start 85.852 86.614) (end 84.813 86.614) (width 0.25) (layer F.Cu) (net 2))
 (segment (start 84.79 92.329) (end 84.813 92.352) (width 0.15) (layer F.Cu) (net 2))
 (segment (start 83.058 92.329) (end 84.79 92.329) (width 0.15) (layer F.Cu) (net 2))
 (segment (start 83.058 90.297) (end 83.058 92.329) (width 0.15) (layer F.Cu) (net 2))
 (segment (start 84.813 92.352) (end 84.813 92.225) (width 0.15) (layer F.Cu) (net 2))
 (segment (start 84.813 92.964) (end 84.813 92.352) (width 0.15) (layer F.Cu) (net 2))
 (segment (start 79.15 88.7) (end 79.429 88.7) (width 0.15) (layer F.Cu) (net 2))
 (segment (start 79.429 88.7) (end 79.45399 88.72499) (width 0.15) (layer F.Cu) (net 2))
 (segment (start 79.45399 88.72499) (end 81.48599 88.72499) (width 0.15) (layer F.Cu) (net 2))
 (segment (start 81.48599 88.72499) (end 83.058 90.297) (width 0.15) (layer F.Cu) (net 2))
 (segment (start 76.4 88.7) (end 76.2 88.9) (width 0.15) (layer F.Cu) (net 2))
 (segment (start 79.15 88.7) (end 76.4 88.7) (width 0.15) (layer F.Cu) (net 2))
 (segment (start 83.843 86.614) (end 83.663002 86.614) (width 0.15) (layer F.Cu) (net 3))
 (segment (start 83.843 86.614) (end 80.899 86.614) (width 0.15) (layer F.Cu) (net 3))
 (segment (start 80.413 87.1) (end 79.15 87.1) (width 0.15) (layer F.Cu) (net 3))
 (segment (start 80.899 86.614) (end 80.413 87.1) (width 0.15) (layer F.Cu) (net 3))
 (segment (start 74.8 85.95) (end 74.8 83.315) (width 0.1) (layer F.Cu) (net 4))
 (segment (start 74.93 83.185) (end 74.93 82.55) (width 0.1) (layer F.Cu) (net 4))
 (segment (start 74.8 83.315) (end 74.93 83.185) (width 0.1) (layer F.Cu) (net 4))
 (segment (start 74.535 82.55) (end 73.66 82.55) (width 0.1) (layer F.Cu) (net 4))
 (segment (start 74.93 82.55) (end 74.535 82.55) (width 0.1) (layer F.Cu) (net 4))
 (segment (start 83.843 91.694) (end 83.843 90.424) (width 0.15) (layer F.Cu) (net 5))
 (segment (start 79.17499 88.32499) (end 79.15 88.3) (width 0.15) (layer F.Cu) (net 5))
 (segment (start 81.72099 88.32499) (end 79.17499 88.32499) (width 0.15) (layer F.Cu) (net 5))
 (segment (start 83.312 89.916) (end 83.058 89.662) (width 0.15) (layer F.Cu) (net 5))
 (segment (start 83.755 89.916) (end 83.312 89.916) (width 0.15) (layer F.Cu) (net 5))
 (segment (start 83.843 90.424) (end 83.843 90.004) (width 0.15) (layer F.Cu) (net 5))
 (segment (start 83.843 90.004) (end 83.755 89.916) (width 0.15) (layer F.Cu) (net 5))
 (segment (start 73.23701 86.72499) (end 71.51701 86.72499) (width 0.15) (layer F.Cu) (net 5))
 (segment (start 73.25 86.7) (end 73.25 86.712) (width 0.15) (layer F.Cu) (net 5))
 (segment (start 73.25 86.712) (end 73.23701 86.72499) (width 0.15) (layer F.Cu) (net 5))
 (segment (start 71.51701 86.72499) (end 71.51701 86.72499) (width 0.15) (layer F.Cu) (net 5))
 (via (at 71.51701 86.72499) (size 0.25) (drill 0.2) (layers F.Cu B.Cu) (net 5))
 (segment (start 83.058 89.662) (end 81.72099 88.32499) (width 0.15) (layer F.Cu) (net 5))
 (via (at 83.058 89.662) (size 0.25) (drill 0.2) (layers F.Cu B.Cu) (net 5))
 (segment (start 71.51701 86.72499) (end 71.51701 84.43899) (width 0.15) (layer B.Cu) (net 5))
 (segment (start 71.51701 84.43899) (end 71.628 84.328) (width 0.15) (layer B.Cu) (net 5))
 (segment (start 77.724 84.328) (end 83.058 89.662) (width 0.15) (layer B.Cu) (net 5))
 (segment (start 71.628 84.328) (end 77.724 84.328) (width 0.15) (layer B.Cu) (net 5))
 (segment (start 72.898 92.952) (end 74 91.85) (width 0.15) (layer F.Cu) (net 6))
 (segment (start 72.517 92.964) (end 72.898 92.964) (width 0.15) (layer F.Cu) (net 6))
 (segment (start 74 85.176) (end 73.914 85.09) (width 0.15) (layer F.Cu) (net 6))
 (segment (start 74 85.95) (end 74 85.176) (width 0.15) (layer F.Cu) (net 6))
 (segment (start 72.898 92.964) (end 72.898 92.952) (width 0.15) (layer F.Cu) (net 6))
 (segment (start 72.263 85.09) (end 72.136 85.217) (width 0.15) (layer F.Cu) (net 6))
 (segment (start 73.914 85.09) (end 72.263 85.09) (width 0.15) (layer F.Cu) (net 6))
 (segment (start 72.136 85.217) (end 72.136 85.217) (width 0.15) (layer F.Cu) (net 6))
 (via (at 72.136 85.217) (size 0.25) (drill 0.2) (layers F.Cu B.Cu) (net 6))
 (segment (start 72.517 92.964) (end 72.136 92.964) (width 0.15) (layer F.Cu) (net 6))
 (segment (start 72.136 92.964) (end 72.136 92.964) (width 0.15) (layer F.Cu) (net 6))
 (via (at 72.136 92.964) (size 0.25) (drill 0.2) (layers F.Cu B.Cu) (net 6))
 (segment (start 72.136 92.964) (end 72.136 85.217) (width 0.15) (layer B.Cu) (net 6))
 (segment (start 79.65 87.9) (end 79.15 87.9) (width 0.15) (layer F.Cu) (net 7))
 (segment (start 81.931 87.9) (end 79.15 87.9) (width 0.15) (layer F.Cu) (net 7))
 (segment (start 83.843 89.154) (end 83.185 89.154) (width 0.15) (layer F.Cu) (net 7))
 (segment (start 83.185 89.154) (end 81.931 87.9) (width 0.15) (layer F.Cu) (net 7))
 (segment (start 83.843 94.234) (end 83.843 92.964) (width 0.15) (layer F.Cu) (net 8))
 (segment (start 79.17301 89.12301) (end 79.15 89.1) (width 0.15) (layer F.Cu) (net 8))
 (segment (start 81.366012 89.1) (end 79.15 89.1) (width 0.15) (layer F.Cu) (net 8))
 (segment (start 82.677 90.410988) (end 81.366012 89.1) (width 0.15) (layer F.Cu) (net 8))
 (segment (start 82.677 92.442988) (end 82.677 90.410988) (width 0.15) (layer F.Cu) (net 8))
 (segment (start 83.843 92.964) (end 83.198012 92.964) (width 0.15) (layer F.Cu) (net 8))
 (segment (start 83.198012 92.964) (end 82.677 92.442988) (width 0.15) (layer F.Cu) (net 8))
 (segment (start 74.4 85.95) (end 74.4 84.56) (width 0.1) (layer F.Cu) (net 10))
 (segment (start 74.145 84.305) (end 72.39 84.305) (width 0.1) (layer F.Cu) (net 10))
 (segment (start 74.4 84.56) (end 74.145 84.305) (width 0.1) (layer F.Cu) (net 10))
 (segment (start 73.475 83.335) (end 73.66 83.52) (width 0.25) (layer F.Cu) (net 11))
 (segment (start 72.575 83.52) (end 72.39 83.335) (width 0.1) (layer F.Cu) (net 11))
 (segment (start 73.66 83.52) (end 72.575 83.52) (width 0.1) (layer F.Cu) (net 11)))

